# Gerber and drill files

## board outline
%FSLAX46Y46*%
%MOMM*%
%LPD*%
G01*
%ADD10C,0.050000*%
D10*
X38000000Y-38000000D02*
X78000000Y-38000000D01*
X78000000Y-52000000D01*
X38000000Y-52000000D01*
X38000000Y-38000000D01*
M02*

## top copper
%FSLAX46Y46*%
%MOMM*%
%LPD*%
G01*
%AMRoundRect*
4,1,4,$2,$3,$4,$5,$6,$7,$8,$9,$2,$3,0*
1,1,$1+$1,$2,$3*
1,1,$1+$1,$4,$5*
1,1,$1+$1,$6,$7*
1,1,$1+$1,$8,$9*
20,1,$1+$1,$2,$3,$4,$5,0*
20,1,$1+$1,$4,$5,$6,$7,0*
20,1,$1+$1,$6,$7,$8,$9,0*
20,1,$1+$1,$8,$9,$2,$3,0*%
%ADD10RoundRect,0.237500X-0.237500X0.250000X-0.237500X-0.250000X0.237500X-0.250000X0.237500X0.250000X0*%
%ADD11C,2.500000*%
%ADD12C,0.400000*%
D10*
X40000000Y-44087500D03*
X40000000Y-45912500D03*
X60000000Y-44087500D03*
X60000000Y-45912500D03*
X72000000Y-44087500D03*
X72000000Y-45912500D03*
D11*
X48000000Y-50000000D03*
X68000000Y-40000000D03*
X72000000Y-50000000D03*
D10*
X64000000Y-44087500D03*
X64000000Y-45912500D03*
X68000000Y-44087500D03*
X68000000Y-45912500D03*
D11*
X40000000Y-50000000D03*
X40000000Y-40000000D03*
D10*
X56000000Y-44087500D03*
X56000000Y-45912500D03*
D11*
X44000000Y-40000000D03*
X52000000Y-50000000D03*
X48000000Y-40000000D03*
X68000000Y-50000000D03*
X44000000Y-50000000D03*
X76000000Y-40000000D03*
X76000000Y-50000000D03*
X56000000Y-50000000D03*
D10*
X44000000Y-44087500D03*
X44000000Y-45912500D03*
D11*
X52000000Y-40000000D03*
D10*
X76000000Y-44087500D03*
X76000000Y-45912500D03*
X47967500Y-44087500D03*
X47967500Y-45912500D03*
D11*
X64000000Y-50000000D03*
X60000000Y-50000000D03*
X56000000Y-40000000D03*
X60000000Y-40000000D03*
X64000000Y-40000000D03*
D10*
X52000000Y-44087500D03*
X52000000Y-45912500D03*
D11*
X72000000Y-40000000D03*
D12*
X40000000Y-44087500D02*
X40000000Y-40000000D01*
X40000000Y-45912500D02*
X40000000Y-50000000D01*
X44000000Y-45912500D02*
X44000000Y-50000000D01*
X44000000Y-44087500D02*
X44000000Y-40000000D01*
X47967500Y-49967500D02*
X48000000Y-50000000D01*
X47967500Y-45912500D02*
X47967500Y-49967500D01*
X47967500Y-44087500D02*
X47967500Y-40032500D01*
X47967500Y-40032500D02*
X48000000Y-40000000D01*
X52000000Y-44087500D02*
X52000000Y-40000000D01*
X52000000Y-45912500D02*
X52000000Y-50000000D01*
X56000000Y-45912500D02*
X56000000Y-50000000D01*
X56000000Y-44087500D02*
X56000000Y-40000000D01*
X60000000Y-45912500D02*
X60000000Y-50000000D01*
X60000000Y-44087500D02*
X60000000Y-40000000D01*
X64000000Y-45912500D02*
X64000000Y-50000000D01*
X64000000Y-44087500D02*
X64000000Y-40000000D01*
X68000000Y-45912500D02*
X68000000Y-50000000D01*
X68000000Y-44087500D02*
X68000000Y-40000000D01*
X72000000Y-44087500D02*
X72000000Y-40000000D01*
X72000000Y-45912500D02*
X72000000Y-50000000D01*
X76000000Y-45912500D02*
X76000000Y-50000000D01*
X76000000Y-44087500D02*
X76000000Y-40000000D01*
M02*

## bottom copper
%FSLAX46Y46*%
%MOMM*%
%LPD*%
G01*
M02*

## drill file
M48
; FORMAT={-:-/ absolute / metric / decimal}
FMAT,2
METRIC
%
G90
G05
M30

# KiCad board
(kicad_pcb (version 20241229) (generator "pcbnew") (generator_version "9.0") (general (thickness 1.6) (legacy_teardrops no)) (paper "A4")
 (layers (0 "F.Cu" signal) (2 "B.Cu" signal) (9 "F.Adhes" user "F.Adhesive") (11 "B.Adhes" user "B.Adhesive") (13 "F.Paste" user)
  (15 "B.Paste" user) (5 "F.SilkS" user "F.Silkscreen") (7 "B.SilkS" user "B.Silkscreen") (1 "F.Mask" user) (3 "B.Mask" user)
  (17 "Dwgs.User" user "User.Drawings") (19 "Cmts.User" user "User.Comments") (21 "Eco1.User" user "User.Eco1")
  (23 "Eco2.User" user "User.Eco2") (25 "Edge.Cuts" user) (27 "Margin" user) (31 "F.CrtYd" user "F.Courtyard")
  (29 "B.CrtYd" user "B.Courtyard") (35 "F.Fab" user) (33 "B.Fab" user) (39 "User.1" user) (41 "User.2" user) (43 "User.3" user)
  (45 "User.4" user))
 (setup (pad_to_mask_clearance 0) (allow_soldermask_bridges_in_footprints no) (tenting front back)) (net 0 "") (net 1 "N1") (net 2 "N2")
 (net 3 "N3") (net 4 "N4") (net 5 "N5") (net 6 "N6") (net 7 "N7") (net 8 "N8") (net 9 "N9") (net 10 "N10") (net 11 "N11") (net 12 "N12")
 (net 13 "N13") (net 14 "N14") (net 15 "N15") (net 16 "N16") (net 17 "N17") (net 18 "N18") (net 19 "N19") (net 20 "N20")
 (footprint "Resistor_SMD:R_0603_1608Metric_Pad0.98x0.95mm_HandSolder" (layer "F.Cu") (at 40 45 -90)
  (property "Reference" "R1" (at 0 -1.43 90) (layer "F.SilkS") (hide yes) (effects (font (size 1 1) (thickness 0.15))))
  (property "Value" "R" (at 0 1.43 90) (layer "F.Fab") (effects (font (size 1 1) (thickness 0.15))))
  (pad "1" smd roundrect (at -0.9125 0 270) (size 0.975 0.95) (layers "F.Cu" "F.Mask" "F.Paste") (roundrect_rratio 0.25) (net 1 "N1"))
  (pad "2" smd roundrect (at 0.9125 0 270) (size 0.975 0.95) (layers "F.Cu" "F.Mask" "F.Paste") (roundrect_rratio 0.25) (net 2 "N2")))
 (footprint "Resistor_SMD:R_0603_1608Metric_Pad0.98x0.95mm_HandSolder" (layer "F.Cu") (at 60 45 -90)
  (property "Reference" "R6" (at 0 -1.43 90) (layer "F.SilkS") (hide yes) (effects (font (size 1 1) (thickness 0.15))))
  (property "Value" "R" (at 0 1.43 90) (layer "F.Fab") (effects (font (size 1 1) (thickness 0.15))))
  (pad "1" smd roundrect (at -0.9125 0 270) (size 0.975 0.95) (layers "F.Cu" "F.Mask" "F.Paste") (roundrect_rratio 0.25) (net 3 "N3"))
  (pad "2" smd roundrect (at 0.9125 0 270) (size 0.975 0.95) (layers "F.Cu" "F.Mask" "F.Paste") (roundrect_rratio 0.25) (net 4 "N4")))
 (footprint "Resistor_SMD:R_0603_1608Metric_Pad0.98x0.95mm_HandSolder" (layer "F.Cu") (at 72 45 -90)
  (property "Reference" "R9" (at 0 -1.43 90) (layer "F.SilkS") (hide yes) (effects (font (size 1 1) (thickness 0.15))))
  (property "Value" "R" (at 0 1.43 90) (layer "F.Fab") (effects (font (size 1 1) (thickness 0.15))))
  (pad "1" smd roundrect (at -0.9125 0 270) (size 0.975 0.95) (layers "F.Cu" "F.Mask" "F.Paste") (roundrect_rratio 0.25) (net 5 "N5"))
  (pad "2" smd roundrect (at 0.9125 0 270) (size 0.975 0.95) (layers "F.Cu" "F.Mask" "F.Paste") (roundrect_rratio 0.25) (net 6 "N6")))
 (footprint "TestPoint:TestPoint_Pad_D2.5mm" (layer "F.Cu") (at 48 50)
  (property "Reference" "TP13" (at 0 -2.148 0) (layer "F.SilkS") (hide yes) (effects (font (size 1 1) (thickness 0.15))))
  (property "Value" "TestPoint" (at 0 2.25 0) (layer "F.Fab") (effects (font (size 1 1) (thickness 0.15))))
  (pad "1" smd circle (at 0 0) (size 2.5 2.5) (layers "F.Cu" "F.Mask") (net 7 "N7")))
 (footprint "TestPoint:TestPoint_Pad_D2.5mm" (layer "F.Cu") (at 68 40)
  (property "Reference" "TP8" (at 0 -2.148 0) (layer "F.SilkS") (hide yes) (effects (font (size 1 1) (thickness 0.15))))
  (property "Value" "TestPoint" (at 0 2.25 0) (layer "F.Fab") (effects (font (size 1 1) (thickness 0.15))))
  (pad "1" smd circle (at 0 0) (size 2.5 2.5) (layers "F.Cu" "F.Mask") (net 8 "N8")))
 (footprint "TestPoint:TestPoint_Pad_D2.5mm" (layer "F.Cu") (at 72 50)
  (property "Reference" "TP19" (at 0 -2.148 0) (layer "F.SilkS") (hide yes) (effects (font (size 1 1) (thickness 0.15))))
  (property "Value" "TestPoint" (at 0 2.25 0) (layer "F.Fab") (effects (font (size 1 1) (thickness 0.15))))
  (pad "1" smd circle (at 0 0) (size 2.5 2.5) (layers "F.Cu" "F.Mask") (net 6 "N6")))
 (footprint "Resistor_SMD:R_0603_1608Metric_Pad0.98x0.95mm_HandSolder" (layer "F.Cu") (at 64 45 -90)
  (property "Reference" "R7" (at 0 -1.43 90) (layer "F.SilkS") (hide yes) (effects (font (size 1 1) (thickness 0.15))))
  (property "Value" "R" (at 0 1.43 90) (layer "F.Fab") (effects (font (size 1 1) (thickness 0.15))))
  (pad "1" smd roundrect (at -0.9125 0 270) (size 0.975 0.95) (layers "F.Cu" "F.Mask" "F.Paste") (roundrect_rratio 0.25) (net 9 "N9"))
  (pad "2" smd roundrect (at 0.9125 0 270) (size 0.975 0.95) (layers "F.Cu" "F.Mask" "F.Paste") (roundrect_rratio 0.25) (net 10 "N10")))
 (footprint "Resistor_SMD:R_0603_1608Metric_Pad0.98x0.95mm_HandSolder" (layer "F.Cu") (at 68 45 -90)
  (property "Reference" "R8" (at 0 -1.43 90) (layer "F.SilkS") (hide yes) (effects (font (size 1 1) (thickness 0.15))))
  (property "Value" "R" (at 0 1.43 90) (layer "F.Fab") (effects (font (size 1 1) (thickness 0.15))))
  (pad "1" smd roundrect (at -0.9125 0 270) (size 0.975 0.95) (layers "F.Cu" "F.Mask" "F.Paste") (roundrect_rratio 0.25) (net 8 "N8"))
  (pad "2" smd roundrect (at 0.9125 0 270) (size 0.975 0.95) (layers "F.Cu" "F.Mask" "F.Paste") (roundrect_rratio 0.25) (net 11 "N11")))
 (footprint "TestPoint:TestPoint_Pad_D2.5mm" (layer "F.Cu") (at 40 50)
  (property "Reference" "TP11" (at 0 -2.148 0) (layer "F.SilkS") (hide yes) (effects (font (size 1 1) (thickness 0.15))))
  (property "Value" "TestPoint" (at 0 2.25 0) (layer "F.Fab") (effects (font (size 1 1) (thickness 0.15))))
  (pad "1" smd circle (at 0 0) (size 2.5 2.5) (layers "F.Cu" "F.Mask") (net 2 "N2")))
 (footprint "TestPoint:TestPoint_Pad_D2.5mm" (layer "F.Cu") (at 40 40)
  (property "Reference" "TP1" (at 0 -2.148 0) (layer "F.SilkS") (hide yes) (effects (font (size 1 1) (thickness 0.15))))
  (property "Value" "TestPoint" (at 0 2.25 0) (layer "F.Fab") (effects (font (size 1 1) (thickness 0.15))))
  (pad "1" smd circle (at 0 0) (size 2.5 2.5) (layers "F.Cu" "F.Mask") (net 1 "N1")))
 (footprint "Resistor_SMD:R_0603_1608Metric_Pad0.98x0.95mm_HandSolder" (layer "F.Cu") (at 56 45 -90)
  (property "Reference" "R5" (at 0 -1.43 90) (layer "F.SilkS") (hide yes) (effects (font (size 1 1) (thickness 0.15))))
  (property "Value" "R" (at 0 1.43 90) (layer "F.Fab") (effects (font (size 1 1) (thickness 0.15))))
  (pad "1" smd roundrect (at -0.9125 0 270) (size 0.975 0.95) (layers "F.Cu" "F.Mask" "F.Paste") (roundrect_rratio 0.25) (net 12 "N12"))
  (pad "2" smd roundrect (at 0.9125 0 270) (size 0.975 0.95) (layers "F.Cu" "F.Mask" "F.Paste") (roundrect_rratio 0.25) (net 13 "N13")))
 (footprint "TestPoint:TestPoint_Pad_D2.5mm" (layer "F.Cu") (at 44 40)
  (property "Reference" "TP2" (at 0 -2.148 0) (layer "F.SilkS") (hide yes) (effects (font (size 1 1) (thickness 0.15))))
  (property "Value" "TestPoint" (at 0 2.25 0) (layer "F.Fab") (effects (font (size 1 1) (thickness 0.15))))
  (pad "1" smd circle (at 0 0) (size 2.5 2.5) (layers "F.Cu" "F.Mask") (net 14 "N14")))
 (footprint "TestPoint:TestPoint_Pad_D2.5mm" (layer "F.Cu") (at 52 50)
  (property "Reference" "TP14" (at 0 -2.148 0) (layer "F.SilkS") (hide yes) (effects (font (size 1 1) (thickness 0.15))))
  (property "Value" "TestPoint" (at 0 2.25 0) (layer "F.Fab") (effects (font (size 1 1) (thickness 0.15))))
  (pad "1" smd circle (at 0 0) (size 2.5 2.5) (layers "F.Cu" "F.Mask") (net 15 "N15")))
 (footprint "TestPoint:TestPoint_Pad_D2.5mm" (layer "F.Cu") (at 48 40)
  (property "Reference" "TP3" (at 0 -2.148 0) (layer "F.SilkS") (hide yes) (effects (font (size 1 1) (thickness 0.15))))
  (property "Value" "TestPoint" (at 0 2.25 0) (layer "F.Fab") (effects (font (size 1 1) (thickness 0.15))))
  (pad "1" smd circle (at 0 0) (size 2.5 2.5) (layers "F.Cu" "F.Mask") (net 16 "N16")))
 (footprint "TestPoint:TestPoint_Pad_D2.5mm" (layer "F.Cu") (at 68 50)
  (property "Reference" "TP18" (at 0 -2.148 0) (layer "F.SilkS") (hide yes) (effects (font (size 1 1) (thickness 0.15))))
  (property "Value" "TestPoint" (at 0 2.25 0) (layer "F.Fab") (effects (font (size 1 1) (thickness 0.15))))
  (pad "1" smd circle (at 0 0) (size 2.5 2.5) (layers "F.Cu" "F.Mask") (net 11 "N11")))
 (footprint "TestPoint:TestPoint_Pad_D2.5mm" (layer "F.Cu") (at 44 50)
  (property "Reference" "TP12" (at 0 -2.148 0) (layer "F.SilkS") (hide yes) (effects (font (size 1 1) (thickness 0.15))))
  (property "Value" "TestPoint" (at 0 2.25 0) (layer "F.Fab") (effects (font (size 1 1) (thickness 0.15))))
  (pad "1" smd circle (at 0 0) (size 2.5 2.5) (layers "F.Cu" "F.Mask") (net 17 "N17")))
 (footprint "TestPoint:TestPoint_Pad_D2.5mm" (layer "F.Cu") (at 76 40)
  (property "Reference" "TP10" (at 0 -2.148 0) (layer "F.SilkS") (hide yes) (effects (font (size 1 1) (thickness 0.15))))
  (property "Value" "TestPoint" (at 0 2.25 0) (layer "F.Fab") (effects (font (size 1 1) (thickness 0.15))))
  (pad "1" smd circle (at 0 0) (size 2.5 2.5) (layers "F.Cu" "F.Mask") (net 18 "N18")))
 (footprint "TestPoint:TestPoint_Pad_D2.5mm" (layer "F.Cu") (at 76 50)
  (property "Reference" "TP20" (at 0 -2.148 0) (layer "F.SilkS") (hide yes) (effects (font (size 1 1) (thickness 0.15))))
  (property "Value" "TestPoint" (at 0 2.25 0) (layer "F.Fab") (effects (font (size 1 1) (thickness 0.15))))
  (pad "1" smd circle (at 0 0) (size 2.5 2.5) (layers "F.Cu" "F.Mask") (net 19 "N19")))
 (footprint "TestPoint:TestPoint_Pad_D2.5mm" (layer "F.Cu") (at 56 50)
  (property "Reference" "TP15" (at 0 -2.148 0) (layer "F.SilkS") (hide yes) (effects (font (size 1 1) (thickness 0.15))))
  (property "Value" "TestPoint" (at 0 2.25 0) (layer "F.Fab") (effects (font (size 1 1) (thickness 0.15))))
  (pad "1" smd circle (at 0 0) (size 2.5 2.5) (layers "F.Cu" "F.Mask") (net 13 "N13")))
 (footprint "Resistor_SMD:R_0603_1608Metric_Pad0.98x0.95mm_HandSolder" (layer "F.Cu") (at 44 45 -90)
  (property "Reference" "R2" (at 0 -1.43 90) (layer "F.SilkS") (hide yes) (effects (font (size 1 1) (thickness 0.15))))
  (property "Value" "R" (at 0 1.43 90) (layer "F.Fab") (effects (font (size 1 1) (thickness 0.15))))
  (pad "1" smd roundrect (at -0.9125 0 270) (size 0.975 0.95) (layers "F.Cu" "F.Mask" "F.Paste") (roundrect_rratio 0.25) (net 14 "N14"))
  (pad "2" smd roundrect (at 0.9125 0 270) (size 0.975 0.95) (layers "F.Cu" "F.Mask" "F.Paste") (roundrect_rratio 0.25) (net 17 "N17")))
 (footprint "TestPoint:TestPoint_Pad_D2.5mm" (layer "F.Cu") (at 52 40)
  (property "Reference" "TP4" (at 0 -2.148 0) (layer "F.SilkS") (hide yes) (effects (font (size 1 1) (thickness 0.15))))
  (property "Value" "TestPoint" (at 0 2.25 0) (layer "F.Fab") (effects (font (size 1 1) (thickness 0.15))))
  (pad "1" smd circle (at 0 0) (size 2.5 2.5) (layers "F.Cu" "F.Mask") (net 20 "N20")))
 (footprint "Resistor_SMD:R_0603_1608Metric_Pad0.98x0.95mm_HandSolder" (layer "F.Cu") (at 76 45 -90)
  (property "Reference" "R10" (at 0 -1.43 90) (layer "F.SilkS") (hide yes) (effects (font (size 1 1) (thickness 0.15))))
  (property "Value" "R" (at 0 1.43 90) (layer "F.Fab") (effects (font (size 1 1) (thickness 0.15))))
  (pad "1" smd roundrect (at -0.9125 0 270) (size 0.975 0.95) (layers "F.Cu" "F.Mask" "F.Paste") (roundrect_rratio 0.25) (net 18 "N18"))
  (pad "2" smd roundrect (at 0.9125 0 270) (size 0.975 0.95) (layers "F.Cu" "F.Mask" "F.Paste") (roundrect_rratio 0.25) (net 19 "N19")))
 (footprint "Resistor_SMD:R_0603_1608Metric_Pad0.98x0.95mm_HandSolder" (layer "F.Cu") (at 47.9675 45 -90)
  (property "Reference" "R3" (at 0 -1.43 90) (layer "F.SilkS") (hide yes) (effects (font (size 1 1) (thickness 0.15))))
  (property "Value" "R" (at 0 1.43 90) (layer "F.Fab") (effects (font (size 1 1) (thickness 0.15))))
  (pad "1" smd roundrect (at -0.9125 0 270) (size 0.975 0.95) (layers "F.Cu" "F.Mask" "F.Paste") (roundrect_rratio 0.25) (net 16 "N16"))
  (pad "2" smd roundrect (at 0.9125 0 270) (size 0.975 0.95) (layers "F.Cu" "F.Mask" "F.Paste") (roundrect_rratio 0.25) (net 7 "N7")))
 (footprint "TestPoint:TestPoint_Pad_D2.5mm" (layer "F.Cu") (at 64 50)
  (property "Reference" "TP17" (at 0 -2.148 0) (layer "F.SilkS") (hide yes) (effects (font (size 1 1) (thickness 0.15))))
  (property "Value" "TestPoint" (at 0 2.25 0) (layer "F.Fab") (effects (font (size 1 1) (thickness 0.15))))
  (pad "1" smd circle (at 0 0) (size 2.5 2.5) (layers "F.Cu" "F.Mask") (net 10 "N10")))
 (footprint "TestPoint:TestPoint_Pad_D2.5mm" (layer "F.Cu") (at 60 50)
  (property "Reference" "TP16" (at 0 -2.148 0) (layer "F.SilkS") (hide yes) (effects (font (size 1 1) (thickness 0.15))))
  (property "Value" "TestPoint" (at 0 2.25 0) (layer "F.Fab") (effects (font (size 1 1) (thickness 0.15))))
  (pad "1" smd circle (at 0 0) (size 2.5 2.5) (layers "F.Cu" "F.Mask") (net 4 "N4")))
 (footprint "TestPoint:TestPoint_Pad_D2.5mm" (layer "F.Cu") (at 56 40)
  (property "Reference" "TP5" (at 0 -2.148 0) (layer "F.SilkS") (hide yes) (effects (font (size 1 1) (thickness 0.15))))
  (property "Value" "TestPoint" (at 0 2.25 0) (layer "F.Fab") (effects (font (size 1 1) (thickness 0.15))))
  (pad "1" smd circle (at 0 0) (size 2.5 2.5) (layers "F.Cu" "F.Mask") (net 12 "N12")))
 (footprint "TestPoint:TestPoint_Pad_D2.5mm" (layer "F.Cu") (at 60 40)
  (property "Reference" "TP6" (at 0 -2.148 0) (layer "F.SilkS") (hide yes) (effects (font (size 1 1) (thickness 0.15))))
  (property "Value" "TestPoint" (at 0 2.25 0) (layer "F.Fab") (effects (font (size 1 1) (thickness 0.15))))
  (pad "1" smd circle (at 0 0) (size 2.5 2.5) (layers "F.Cu" "F.Mask") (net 3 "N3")))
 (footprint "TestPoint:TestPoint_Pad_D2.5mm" (layer "F.Cu") (at 64 40)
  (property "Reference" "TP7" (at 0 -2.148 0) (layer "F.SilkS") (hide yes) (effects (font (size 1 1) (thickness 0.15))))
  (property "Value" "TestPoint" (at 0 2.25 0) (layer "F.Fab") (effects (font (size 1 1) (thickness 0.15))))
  (pad "1" smd circle (at 0 0) (size 2.5 2.5) (layers "F.Cu" "F.Mask") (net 9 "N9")))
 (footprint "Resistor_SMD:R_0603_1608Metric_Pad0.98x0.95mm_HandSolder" (layer "F.Cu") (at 52 45 -90)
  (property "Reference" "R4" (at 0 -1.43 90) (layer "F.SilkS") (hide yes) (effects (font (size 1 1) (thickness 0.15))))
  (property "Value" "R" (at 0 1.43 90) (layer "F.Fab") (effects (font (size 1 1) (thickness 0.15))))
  (pad "1" smd roundrect (at -0.9125 0 270) (size 0.975 0.95) (layers "F.Cu" "F.Mask" "F.Paste") (roundrect_rratio 0.25) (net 20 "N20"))
  (pad "2" smd roundrect (at 0.9125 0 270) (size 0.975 0.95) (layers "F.Cu" "F.Mask" "F.Paste") (roundrect_rratio 0.25) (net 15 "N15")))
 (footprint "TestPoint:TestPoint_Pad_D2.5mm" (layer "F.Cu") (at 72 40)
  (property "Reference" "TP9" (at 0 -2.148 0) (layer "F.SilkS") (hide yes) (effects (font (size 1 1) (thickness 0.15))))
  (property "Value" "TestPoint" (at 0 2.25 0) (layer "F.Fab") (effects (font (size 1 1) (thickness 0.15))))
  (pad "1" smd circle (at 0 0) (size 2.5 2.5) (layers "F.Cu" "F.Mask") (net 5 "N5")))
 (gr_rect (start 38 38) (end 78 52) (stroke (width 0.05) (type default)) (fill no) (layer "Edge.Cuts"))
 (segment (start 40 44.0875) (end 40 40) (width 0.4) (layer "F.Cu") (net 1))
 (segment (start 40 45.9125) (end 40 50) (width 0.4) (layer "F.Cu") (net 2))
 (segment (start 44 45.9125) (end 44 50) (width 0.4) (layer "F.Cu") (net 17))
 (segment (start 44 44.0875) (end 44 40) (width 0.4) (layer "F.Cu") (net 14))
 (segment (start 47.9675 49.9675) (end 48 50) (width 0.4) (layer "F.Cu") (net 7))
 (segment (start 47.9675 45.9125) (end 47.9675 49.9675) (width 0.4) (layer "F.Cu") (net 7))
 (segment (start 47.9675 44.0875) (end 47.9675 40.0325) (width 0.4) (layer "F.Cu") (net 16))
 (segment (start 47.9675 40.0325) (end 48 40) (width 0.4) (layer "F.Cu") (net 16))
 (segment (start 52 44.0875) (end 52 40) (width 0.4) (layer "F.Cu") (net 20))
 (segment (start 52 45.9125) (end 52 50) (width 0.4) (layer "F.Cu") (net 15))
 (segment (start 56 45.9125) (end 56 50) (width 0.4) (layer "F.Cu") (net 13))
 (segment (start 56 44.0875) (end 56 40) (width 0.4) (layer "F.Cu") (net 12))
 (segment (start 60 45.9125) (end 60 50) (width 0.4) (layer "F.Cu") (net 4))
 (segment (start 60 44.0875) (end 60 40) (width 0.4) (layer "F.Cu") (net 3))
 (segment (start 64 45.9125) (end 64 50) (width 0.4) (layer "F.Cu") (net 10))
 (segment (start 64 44.0875) (end 64 40) (width 0.4) (layer "F.Cu") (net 9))
 (segment (start 68 45.9125) (end 68 50) (width 0.4) (layer "F.Cu") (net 11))
 (segment (start 68 44.0875) (end 68 40) (width 0.4) (layer "F.Cu") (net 8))
 (segment (start 72 44.0875) (end 72 40) (width 0.4) (layer "F.Cu") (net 5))
 (segment (start 72 45.9125) (end 72 50) (width 0.4) (layer "F.Cu") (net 6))
 (segment (start 76 45.9125) (end 76 50) (width 0.4) (layer "F.Cu") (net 19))
 (segment (start 76 44.0875) (end 76 40) (width 0.4) (layer "F.Cu") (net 18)))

